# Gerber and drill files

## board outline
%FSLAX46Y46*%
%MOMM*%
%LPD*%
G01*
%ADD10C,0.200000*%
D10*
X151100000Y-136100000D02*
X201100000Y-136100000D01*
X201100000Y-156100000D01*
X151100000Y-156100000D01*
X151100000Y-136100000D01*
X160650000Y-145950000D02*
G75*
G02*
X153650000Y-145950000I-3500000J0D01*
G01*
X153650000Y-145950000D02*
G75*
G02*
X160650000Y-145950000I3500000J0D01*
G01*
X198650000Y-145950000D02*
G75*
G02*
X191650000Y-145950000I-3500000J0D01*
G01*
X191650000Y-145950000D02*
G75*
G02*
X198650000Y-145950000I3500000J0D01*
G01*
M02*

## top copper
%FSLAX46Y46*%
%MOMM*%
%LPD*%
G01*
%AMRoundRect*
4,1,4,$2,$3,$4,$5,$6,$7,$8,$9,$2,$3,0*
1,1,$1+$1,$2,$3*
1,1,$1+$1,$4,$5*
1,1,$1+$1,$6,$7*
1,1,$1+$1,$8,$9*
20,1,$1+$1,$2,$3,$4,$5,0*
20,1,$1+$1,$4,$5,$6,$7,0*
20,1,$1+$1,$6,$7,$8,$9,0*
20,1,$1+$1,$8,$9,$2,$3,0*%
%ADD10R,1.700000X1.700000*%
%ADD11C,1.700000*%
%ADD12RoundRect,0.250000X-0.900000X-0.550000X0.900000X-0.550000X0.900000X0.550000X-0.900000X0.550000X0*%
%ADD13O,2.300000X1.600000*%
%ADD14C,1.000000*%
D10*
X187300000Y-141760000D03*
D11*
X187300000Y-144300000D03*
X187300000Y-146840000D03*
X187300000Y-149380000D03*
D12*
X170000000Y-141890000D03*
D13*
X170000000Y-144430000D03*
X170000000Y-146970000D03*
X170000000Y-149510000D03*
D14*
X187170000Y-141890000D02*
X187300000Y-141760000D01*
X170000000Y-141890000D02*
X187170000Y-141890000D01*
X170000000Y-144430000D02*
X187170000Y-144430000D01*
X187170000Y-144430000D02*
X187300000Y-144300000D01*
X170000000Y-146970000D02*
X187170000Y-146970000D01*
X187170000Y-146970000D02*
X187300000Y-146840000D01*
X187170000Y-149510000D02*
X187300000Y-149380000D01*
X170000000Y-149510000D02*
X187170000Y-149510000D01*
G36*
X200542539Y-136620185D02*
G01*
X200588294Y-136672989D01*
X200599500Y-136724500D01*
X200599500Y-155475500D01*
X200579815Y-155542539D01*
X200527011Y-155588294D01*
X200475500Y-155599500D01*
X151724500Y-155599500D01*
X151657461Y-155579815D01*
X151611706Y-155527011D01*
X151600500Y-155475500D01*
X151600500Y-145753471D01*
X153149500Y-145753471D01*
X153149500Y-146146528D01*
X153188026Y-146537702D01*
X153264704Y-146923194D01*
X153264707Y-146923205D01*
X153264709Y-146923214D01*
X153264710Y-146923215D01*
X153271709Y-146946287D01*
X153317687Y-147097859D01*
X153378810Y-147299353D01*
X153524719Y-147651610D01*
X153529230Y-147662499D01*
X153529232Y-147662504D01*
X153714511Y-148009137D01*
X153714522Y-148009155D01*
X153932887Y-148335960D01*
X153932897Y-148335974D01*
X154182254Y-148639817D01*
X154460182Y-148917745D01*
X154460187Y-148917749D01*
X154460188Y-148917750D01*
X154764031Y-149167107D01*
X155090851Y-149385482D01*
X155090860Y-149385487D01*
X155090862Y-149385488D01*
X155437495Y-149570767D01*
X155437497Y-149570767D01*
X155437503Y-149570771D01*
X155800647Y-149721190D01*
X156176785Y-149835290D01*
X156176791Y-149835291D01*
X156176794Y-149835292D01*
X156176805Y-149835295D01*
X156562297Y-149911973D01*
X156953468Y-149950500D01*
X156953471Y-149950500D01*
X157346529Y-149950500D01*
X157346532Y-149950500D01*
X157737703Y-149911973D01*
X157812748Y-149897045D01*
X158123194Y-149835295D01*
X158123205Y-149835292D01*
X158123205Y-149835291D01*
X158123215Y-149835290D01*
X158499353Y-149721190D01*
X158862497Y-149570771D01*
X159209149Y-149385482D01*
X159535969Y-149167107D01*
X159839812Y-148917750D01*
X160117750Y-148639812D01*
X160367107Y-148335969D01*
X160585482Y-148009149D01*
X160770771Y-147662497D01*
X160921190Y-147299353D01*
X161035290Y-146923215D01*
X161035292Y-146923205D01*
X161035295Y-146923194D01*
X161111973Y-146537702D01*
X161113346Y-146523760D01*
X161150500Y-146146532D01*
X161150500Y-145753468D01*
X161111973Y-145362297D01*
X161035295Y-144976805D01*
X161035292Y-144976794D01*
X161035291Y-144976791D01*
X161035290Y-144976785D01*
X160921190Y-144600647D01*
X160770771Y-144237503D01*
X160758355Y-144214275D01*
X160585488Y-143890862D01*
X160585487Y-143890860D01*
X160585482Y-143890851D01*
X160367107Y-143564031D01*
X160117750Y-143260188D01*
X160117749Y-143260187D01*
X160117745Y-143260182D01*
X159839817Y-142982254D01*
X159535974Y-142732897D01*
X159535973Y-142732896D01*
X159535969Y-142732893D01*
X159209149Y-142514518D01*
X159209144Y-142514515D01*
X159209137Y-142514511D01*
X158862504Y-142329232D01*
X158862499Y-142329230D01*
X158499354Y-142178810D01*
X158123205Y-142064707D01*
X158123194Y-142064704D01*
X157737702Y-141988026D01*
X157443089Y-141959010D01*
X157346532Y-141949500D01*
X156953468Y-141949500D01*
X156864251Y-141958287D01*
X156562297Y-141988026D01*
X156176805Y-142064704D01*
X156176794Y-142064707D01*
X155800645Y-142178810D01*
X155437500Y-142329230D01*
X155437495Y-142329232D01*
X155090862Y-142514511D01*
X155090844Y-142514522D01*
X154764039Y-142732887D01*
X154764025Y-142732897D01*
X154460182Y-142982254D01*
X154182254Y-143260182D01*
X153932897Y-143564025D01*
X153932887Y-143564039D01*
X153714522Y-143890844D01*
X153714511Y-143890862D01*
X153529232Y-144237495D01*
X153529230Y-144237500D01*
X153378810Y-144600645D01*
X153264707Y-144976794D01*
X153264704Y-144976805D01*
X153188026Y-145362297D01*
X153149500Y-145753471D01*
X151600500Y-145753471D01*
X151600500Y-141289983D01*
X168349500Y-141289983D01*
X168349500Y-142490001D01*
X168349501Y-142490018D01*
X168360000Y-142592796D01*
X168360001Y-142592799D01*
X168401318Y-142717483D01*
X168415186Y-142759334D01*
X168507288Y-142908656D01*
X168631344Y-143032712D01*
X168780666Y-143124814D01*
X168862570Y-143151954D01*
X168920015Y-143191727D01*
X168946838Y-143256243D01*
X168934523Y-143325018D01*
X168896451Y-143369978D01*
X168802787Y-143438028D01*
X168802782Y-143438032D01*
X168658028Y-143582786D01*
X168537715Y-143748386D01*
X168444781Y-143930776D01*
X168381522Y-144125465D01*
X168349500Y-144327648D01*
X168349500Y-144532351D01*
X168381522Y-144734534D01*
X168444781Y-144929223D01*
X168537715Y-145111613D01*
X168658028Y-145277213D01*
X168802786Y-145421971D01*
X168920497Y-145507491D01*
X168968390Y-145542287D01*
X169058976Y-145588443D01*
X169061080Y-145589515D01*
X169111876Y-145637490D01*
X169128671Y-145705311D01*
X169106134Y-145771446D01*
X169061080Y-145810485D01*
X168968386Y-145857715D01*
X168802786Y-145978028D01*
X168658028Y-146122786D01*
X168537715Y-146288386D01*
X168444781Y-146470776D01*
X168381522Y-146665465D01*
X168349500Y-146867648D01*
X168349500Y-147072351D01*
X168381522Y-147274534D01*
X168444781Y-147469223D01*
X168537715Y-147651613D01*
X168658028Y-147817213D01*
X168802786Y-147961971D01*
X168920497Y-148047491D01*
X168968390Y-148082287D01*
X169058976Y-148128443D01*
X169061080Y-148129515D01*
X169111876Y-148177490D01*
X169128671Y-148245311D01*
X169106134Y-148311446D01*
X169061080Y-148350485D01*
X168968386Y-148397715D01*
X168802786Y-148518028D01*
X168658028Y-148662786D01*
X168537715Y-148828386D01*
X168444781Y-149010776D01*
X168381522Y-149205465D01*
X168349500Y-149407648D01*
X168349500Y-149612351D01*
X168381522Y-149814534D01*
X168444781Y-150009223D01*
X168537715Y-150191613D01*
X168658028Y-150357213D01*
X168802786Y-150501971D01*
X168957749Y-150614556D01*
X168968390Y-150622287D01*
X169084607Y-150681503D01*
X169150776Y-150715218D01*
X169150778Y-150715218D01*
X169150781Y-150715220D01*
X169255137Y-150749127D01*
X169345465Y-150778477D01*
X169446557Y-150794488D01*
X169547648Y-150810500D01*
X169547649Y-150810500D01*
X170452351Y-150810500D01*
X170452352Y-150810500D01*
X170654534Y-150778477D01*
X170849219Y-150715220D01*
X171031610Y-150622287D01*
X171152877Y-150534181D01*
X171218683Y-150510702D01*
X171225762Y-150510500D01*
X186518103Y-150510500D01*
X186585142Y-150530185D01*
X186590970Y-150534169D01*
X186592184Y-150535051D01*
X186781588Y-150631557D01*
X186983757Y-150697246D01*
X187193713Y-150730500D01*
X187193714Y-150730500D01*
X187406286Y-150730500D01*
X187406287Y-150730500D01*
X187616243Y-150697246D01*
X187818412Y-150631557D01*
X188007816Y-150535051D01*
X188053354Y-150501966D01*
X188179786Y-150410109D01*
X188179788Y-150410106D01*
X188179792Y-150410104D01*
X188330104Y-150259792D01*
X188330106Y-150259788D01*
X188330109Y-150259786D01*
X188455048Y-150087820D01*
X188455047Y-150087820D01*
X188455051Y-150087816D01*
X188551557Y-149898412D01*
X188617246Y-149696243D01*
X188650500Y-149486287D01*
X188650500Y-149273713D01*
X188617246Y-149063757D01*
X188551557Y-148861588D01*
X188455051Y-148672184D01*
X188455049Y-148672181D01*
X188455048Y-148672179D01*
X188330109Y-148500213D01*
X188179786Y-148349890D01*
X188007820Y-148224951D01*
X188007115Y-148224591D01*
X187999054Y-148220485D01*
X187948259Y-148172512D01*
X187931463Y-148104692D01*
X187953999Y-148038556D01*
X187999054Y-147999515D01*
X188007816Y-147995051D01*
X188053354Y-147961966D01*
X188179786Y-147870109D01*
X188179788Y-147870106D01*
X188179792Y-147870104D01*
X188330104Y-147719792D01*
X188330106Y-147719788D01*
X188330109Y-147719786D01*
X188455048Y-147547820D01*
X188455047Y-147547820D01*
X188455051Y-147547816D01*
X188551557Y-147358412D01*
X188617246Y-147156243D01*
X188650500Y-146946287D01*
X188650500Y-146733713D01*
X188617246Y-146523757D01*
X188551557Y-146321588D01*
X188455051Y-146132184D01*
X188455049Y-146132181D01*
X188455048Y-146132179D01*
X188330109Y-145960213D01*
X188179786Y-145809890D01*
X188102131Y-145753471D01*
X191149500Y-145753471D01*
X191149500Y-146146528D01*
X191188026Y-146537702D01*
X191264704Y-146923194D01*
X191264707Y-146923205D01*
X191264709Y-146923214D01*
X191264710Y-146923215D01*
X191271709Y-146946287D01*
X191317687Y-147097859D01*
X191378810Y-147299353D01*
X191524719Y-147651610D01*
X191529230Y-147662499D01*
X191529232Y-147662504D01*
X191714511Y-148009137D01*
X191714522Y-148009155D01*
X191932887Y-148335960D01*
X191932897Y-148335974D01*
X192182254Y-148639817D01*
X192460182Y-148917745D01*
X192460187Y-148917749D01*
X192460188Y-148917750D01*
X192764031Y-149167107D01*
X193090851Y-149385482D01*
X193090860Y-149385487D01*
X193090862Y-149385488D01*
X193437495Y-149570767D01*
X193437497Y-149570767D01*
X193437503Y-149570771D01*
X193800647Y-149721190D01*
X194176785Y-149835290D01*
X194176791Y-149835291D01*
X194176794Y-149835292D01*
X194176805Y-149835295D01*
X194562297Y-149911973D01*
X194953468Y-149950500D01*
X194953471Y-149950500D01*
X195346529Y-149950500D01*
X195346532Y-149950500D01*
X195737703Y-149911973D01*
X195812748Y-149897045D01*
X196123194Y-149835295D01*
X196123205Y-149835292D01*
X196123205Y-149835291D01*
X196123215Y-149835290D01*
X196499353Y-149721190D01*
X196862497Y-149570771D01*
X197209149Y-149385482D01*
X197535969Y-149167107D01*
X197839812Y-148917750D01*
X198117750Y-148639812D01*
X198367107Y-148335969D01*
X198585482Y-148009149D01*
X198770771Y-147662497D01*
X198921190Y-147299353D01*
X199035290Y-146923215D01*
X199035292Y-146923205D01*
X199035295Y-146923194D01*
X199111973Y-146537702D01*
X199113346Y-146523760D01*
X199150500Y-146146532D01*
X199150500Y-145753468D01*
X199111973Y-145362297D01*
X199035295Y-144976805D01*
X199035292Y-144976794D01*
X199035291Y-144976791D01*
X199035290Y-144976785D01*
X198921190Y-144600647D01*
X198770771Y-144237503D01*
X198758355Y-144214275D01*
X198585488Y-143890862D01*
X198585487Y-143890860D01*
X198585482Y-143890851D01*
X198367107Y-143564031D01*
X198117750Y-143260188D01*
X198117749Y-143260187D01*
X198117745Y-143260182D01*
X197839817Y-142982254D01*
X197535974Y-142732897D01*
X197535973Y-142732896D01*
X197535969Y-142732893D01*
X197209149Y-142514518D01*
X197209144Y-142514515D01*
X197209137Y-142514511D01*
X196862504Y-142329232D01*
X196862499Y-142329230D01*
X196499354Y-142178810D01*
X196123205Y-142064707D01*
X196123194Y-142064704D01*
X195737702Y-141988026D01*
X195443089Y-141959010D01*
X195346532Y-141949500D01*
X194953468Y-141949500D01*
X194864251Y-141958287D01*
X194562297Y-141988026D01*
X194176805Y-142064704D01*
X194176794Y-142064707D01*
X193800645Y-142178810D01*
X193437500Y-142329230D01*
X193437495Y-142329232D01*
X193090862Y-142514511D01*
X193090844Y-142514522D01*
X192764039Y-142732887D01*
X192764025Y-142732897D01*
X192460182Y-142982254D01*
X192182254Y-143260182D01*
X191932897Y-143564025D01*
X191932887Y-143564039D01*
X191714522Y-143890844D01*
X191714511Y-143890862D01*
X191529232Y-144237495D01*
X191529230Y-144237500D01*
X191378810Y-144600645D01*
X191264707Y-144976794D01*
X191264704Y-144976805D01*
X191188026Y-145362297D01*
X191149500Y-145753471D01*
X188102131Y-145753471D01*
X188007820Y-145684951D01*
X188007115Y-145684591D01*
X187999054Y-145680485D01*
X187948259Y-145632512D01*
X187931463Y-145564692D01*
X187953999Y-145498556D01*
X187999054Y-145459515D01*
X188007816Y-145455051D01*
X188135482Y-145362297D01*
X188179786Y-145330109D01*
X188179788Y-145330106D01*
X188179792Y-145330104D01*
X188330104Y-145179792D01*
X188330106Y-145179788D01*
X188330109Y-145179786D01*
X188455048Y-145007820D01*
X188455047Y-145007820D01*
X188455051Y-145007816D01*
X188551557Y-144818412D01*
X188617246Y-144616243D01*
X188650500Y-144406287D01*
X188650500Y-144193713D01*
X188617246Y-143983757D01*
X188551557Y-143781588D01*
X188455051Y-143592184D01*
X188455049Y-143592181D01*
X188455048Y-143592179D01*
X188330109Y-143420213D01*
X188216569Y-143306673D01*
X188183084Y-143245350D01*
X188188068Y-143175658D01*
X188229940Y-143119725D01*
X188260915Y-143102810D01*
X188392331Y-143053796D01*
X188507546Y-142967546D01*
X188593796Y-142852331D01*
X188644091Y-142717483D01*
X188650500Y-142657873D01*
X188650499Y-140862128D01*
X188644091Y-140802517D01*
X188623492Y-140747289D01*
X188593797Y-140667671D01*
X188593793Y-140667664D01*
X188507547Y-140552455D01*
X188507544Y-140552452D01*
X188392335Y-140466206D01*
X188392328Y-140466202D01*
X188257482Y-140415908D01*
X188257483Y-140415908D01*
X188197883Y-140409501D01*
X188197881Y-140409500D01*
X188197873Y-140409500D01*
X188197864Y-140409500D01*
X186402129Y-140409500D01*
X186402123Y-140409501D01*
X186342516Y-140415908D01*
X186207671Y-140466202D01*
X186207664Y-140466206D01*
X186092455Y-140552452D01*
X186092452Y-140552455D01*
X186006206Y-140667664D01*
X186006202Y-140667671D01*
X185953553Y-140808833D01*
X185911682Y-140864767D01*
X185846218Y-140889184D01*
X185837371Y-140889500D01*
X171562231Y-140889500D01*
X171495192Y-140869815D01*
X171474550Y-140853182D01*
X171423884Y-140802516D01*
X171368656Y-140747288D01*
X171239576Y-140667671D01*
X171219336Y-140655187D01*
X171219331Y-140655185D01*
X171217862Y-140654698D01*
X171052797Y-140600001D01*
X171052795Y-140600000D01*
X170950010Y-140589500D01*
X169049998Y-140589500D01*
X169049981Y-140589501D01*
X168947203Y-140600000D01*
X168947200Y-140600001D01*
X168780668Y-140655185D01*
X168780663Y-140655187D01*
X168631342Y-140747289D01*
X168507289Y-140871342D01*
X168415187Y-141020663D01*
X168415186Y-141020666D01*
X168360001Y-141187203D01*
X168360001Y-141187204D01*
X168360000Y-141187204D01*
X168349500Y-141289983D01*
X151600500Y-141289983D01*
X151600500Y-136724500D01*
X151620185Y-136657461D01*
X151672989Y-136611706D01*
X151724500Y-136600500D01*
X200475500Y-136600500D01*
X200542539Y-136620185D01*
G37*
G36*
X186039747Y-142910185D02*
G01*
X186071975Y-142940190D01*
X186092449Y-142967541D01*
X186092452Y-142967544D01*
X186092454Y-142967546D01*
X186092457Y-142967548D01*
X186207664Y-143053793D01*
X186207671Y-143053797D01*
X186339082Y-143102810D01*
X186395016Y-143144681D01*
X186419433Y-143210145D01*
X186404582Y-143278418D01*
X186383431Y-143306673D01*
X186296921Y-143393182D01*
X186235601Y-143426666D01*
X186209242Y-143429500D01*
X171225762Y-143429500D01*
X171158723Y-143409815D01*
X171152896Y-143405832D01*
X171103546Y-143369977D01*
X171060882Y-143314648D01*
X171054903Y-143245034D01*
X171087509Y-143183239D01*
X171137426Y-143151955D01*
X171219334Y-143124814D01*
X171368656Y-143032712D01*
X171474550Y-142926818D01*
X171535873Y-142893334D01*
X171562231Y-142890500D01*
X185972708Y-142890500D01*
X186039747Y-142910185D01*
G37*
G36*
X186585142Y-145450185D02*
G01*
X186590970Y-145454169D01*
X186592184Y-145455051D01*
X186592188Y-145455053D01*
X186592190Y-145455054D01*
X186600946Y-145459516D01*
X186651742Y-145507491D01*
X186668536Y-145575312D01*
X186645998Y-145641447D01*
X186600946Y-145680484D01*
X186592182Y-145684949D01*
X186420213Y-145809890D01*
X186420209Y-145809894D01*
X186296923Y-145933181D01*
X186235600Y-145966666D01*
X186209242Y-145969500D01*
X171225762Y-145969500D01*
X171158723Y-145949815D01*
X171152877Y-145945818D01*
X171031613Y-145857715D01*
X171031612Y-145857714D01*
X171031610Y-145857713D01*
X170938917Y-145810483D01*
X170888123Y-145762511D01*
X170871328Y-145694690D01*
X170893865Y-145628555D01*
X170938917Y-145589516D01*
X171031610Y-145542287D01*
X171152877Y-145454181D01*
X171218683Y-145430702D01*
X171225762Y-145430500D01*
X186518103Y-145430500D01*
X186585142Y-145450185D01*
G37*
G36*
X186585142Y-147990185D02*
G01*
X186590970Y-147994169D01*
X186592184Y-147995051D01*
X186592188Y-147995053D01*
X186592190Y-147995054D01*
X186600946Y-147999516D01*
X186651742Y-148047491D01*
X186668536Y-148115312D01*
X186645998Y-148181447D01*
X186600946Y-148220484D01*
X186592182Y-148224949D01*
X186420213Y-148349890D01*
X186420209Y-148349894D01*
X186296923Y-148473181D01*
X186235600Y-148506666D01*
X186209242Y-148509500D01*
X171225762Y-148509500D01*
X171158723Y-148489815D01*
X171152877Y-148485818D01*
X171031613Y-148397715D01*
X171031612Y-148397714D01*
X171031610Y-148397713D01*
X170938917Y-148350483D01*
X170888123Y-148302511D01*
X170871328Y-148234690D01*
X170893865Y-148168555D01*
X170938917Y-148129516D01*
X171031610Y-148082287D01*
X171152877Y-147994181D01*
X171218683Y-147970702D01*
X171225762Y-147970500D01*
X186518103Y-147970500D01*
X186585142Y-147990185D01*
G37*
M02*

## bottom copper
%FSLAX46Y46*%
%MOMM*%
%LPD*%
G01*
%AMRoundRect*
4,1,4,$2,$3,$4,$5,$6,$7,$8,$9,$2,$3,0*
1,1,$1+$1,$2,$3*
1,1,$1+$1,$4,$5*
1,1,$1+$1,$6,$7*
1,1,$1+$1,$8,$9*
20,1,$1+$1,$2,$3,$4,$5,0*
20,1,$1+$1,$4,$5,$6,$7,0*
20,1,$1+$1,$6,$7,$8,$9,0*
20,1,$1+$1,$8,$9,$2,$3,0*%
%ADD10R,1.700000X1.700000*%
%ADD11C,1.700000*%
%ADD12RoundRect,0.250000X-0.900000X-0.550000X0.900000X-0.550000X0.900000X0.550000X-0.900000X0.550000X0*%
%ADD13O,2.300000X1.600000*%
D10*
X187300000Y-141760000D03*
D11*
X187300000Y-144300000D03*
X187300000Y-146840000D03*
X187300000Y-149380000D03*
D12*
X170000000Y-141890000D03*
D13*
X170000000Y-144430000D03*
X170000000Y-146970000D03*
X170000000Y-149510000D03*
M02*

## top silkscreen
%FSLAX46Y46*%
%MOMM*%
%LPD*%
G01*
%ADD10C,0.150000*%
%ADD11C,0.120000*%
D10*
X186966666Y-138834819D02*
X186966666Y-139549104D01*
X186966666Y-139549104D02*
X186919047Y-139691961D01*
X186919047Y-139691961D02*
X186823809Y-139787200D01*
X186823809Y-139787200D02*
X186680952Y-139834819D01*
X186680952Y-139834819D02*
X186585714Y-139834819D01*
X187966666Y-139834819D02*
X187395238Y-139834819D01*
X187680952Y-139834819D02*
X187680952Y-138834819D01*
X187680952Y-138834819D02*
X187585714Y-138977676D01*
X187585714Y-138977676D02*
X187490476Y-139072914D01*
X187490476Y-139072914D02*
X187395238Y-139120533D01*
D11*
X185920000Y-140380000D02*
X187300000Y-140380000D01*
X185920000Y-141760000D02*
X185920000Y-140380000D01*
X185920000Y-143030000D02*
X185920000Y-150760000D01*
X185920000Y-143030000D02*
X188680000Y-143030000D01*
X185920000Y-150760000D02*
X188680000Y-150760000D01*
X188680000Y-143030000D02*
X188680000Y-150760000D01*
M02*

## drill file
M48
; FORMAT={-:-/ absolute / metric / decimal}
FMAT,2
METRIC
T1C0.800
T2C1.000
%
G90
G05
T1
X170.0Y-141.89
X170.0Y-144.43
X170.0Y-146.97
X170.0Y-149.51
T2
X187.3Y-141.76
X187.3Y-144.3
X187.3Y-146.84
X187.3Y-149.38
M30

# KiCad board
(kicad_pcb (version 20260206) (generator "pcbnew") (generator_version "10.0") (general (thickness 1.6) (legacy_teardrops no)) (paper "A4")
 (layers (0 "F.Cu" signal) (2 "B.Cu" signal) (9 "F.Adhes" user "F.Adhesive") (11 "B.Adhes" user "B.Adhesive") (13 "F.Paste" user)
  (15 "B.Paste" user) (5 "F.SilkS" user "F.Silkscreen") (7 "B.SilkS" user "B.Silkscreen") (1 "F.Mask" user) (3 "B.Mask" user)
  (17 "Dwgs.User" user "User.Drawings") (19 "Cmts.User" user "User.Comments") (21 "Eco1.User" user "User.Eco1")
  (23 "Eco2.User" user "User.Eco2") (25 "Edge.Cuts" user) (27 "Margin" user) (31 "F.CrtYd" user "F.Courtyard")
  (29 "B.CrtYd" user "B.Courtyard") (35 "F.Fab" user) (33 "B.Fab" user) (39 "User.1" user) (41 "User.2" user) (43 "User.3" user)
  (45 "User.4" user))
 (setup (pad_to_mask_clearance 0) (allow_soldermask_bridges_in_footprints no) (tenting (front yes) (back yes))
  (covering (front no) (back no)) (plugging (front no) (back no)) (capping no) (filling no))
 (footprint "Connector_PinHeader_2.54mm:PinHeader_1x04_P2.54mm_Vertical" (layer "F.Cu") (at 187.3 141.76)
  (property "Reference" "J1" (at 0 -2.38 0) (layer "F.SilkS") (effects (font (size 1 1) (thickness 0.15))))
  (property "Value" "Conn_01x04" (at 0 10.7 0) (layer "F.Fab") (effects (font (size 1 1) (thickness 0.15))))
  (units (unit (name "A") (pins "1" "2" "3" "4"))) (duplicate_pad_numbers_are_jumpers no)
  (fp_line (start -1.38 -1.38) (end 0 -1.38) (stroke (width 0.12) (type solid)) (layer "F.SilkS"))
  (fp_line (start -1.38 0) (end -1.38 -1.38) (stroke (width 0.12) (type solid)) (layer "F.SilkS"))
  (fp_line (start -1.38 1.27) (end -1.38 9) (stroke (width 0.12) (type solid)) (layer "F.SilkS"))
  (fp_line (start -1.38 1.27) (end 1.38 1.27) (stroke (width 0.12) (type solid)) (layer "F.SilkS"))
  (fp_line (start -1.38 9) (end 1.38 9) (stroke (width 0.12) (type solid)) (layer "F.SilkS"))
  (fp_line (start 1.38 1.27) (end 1.38 9) (stroke (width 0.12) (type solid)) (layer "F.SilkS"))
  (pad "1" thru_hole rect (at 0 0) (size 1.7 1.7) (drill 1) (layers "*.Cu" "*.Mask") (remove_unused_layers no) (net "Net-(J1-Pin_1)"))
  (pad "2" thru_hole circle (at 0 2.54) (size 1.7 1.7) (drill 1) (layers "*.Cu" "*.Mask") (remove_unused_layers no) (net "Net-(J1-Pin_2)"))
  (pad "3" thru_hole circle (at 0 5.08) (size 1.7 1.7) (drill 1) (layers "*.Cu" "*.Mask") (remove_unused_layers no) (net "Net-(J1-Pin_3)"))
  (pad "4" thru_hole circle (at 0 7.62) (size 1.7 1.7) (drill 1) (layers "*.Cu" "*.Mask") (remove_unused_layers no) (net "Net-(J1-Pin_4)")))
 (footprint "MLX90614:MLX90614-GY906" (layer "F.Cu") (at 176 150.7)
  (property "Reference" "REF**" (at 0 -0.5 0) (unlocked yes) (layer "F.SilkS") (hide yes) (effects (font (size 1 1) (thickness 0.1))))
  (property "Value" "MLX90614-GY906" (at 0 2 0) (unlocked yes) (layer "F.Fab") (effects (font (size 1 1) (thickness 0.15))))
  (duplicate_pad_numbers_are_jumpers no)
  (pad "1" thru_hole roundrect (at -6 -8.81) (size 2.3 1.6) (drill 0.8) (layers "*.Cu" "*.Mask") (remove_unused_layers no)
   (roundrect_rratio 0.15625) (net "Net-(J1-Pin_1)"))
  (pad "2" thru_hole oval (at -6 -6.27) (size 2.3 1.6) (drill 0.8) (layers "*.Cu" "*.Mask") (remove_unused_layers no) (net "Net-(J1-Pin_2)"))
  (pad "3" thru_hole oval (at -6 -3.73) (size 2.3 1.6) (drill 0.8) (layers "*.Cu" "*.Mask") (remove_unused_layers no) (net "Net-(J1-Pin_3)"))
  (pad "4" thru_hole oval (at -6 -1.19) (size 2.3 1.6) (drill 0.8) (layers "*.Cu" "*.Mask") (remove_unused_layers no) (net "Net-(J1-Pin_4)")))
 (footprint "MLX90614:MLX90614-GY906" (layer "F.Cu") (at 176.05 145.95)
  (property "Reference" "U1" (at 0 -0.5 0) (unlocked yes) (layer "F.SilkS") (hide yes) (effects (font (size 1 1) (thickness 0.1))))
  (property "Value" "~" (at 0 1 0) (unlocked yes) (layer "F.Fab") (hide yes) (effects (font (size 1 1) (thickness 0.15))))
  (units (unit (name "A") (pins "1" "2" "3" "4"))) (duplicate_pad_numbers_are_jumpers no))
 (gr_rect (start 151.1 136.1) (end 201.1 156.1) (stroke (width 0.2) (type solid)) (fill no) (layer "Edge.Cuts"))
 (gr_circle (center 157.15 145.95) (end 160.65 145.95) (stroke (width 0.2) (type solid)) (fill no) (layer "Edge.Cuts"))
 (gr_circle (center 195.15 145.95) (end 198.65 145.95) (stroke (width 0.2) (type solid)) (fill no) (layer "Edge.Cuts"))
 (segment (start 187.17 141.89) (end 187.3 141.76) (width 1) (layer "F.Cu") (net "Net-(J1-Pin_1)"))
 (segment (start 170 141.89) (end 187.17 141.89) (width 1) (layer "F.Cu") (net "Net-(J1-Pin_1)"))
 (segment (start 170 144.43) (end 187.17 144.43) (width 1) (layer "F.Cu") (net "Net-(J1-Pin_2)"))
 (segment (start 187.17 144.43) (end 187.3 144.3) (width 1) (layer "F.Cu") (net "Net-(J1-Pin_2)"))
 (segment (start 170 146.97) (end 187.17 146.97) (width 1) (layer "F.Cu") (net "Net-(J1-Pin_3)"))
 (segment (start 187.17 146.97) (end 187.3 146.84) (width 1) (layer "F.Cu") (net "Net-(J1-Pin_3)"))
 (segment (start 187.17 149.51) (end 187.3 149.38) (width 1) (layer "F.Cu") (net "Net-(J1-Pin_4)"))
 (segment (start 170 149.51) (end 187.17 149.51) (width 1) (layer "F.Cu") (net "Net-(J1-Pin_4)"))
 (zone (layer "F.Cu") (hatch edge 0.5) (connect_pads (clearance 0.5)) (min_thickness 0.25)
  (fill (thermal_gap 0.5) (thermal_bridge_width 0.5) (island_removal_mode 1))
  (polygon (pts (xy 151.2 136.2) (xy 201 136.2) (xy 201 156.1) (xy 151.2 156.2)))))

